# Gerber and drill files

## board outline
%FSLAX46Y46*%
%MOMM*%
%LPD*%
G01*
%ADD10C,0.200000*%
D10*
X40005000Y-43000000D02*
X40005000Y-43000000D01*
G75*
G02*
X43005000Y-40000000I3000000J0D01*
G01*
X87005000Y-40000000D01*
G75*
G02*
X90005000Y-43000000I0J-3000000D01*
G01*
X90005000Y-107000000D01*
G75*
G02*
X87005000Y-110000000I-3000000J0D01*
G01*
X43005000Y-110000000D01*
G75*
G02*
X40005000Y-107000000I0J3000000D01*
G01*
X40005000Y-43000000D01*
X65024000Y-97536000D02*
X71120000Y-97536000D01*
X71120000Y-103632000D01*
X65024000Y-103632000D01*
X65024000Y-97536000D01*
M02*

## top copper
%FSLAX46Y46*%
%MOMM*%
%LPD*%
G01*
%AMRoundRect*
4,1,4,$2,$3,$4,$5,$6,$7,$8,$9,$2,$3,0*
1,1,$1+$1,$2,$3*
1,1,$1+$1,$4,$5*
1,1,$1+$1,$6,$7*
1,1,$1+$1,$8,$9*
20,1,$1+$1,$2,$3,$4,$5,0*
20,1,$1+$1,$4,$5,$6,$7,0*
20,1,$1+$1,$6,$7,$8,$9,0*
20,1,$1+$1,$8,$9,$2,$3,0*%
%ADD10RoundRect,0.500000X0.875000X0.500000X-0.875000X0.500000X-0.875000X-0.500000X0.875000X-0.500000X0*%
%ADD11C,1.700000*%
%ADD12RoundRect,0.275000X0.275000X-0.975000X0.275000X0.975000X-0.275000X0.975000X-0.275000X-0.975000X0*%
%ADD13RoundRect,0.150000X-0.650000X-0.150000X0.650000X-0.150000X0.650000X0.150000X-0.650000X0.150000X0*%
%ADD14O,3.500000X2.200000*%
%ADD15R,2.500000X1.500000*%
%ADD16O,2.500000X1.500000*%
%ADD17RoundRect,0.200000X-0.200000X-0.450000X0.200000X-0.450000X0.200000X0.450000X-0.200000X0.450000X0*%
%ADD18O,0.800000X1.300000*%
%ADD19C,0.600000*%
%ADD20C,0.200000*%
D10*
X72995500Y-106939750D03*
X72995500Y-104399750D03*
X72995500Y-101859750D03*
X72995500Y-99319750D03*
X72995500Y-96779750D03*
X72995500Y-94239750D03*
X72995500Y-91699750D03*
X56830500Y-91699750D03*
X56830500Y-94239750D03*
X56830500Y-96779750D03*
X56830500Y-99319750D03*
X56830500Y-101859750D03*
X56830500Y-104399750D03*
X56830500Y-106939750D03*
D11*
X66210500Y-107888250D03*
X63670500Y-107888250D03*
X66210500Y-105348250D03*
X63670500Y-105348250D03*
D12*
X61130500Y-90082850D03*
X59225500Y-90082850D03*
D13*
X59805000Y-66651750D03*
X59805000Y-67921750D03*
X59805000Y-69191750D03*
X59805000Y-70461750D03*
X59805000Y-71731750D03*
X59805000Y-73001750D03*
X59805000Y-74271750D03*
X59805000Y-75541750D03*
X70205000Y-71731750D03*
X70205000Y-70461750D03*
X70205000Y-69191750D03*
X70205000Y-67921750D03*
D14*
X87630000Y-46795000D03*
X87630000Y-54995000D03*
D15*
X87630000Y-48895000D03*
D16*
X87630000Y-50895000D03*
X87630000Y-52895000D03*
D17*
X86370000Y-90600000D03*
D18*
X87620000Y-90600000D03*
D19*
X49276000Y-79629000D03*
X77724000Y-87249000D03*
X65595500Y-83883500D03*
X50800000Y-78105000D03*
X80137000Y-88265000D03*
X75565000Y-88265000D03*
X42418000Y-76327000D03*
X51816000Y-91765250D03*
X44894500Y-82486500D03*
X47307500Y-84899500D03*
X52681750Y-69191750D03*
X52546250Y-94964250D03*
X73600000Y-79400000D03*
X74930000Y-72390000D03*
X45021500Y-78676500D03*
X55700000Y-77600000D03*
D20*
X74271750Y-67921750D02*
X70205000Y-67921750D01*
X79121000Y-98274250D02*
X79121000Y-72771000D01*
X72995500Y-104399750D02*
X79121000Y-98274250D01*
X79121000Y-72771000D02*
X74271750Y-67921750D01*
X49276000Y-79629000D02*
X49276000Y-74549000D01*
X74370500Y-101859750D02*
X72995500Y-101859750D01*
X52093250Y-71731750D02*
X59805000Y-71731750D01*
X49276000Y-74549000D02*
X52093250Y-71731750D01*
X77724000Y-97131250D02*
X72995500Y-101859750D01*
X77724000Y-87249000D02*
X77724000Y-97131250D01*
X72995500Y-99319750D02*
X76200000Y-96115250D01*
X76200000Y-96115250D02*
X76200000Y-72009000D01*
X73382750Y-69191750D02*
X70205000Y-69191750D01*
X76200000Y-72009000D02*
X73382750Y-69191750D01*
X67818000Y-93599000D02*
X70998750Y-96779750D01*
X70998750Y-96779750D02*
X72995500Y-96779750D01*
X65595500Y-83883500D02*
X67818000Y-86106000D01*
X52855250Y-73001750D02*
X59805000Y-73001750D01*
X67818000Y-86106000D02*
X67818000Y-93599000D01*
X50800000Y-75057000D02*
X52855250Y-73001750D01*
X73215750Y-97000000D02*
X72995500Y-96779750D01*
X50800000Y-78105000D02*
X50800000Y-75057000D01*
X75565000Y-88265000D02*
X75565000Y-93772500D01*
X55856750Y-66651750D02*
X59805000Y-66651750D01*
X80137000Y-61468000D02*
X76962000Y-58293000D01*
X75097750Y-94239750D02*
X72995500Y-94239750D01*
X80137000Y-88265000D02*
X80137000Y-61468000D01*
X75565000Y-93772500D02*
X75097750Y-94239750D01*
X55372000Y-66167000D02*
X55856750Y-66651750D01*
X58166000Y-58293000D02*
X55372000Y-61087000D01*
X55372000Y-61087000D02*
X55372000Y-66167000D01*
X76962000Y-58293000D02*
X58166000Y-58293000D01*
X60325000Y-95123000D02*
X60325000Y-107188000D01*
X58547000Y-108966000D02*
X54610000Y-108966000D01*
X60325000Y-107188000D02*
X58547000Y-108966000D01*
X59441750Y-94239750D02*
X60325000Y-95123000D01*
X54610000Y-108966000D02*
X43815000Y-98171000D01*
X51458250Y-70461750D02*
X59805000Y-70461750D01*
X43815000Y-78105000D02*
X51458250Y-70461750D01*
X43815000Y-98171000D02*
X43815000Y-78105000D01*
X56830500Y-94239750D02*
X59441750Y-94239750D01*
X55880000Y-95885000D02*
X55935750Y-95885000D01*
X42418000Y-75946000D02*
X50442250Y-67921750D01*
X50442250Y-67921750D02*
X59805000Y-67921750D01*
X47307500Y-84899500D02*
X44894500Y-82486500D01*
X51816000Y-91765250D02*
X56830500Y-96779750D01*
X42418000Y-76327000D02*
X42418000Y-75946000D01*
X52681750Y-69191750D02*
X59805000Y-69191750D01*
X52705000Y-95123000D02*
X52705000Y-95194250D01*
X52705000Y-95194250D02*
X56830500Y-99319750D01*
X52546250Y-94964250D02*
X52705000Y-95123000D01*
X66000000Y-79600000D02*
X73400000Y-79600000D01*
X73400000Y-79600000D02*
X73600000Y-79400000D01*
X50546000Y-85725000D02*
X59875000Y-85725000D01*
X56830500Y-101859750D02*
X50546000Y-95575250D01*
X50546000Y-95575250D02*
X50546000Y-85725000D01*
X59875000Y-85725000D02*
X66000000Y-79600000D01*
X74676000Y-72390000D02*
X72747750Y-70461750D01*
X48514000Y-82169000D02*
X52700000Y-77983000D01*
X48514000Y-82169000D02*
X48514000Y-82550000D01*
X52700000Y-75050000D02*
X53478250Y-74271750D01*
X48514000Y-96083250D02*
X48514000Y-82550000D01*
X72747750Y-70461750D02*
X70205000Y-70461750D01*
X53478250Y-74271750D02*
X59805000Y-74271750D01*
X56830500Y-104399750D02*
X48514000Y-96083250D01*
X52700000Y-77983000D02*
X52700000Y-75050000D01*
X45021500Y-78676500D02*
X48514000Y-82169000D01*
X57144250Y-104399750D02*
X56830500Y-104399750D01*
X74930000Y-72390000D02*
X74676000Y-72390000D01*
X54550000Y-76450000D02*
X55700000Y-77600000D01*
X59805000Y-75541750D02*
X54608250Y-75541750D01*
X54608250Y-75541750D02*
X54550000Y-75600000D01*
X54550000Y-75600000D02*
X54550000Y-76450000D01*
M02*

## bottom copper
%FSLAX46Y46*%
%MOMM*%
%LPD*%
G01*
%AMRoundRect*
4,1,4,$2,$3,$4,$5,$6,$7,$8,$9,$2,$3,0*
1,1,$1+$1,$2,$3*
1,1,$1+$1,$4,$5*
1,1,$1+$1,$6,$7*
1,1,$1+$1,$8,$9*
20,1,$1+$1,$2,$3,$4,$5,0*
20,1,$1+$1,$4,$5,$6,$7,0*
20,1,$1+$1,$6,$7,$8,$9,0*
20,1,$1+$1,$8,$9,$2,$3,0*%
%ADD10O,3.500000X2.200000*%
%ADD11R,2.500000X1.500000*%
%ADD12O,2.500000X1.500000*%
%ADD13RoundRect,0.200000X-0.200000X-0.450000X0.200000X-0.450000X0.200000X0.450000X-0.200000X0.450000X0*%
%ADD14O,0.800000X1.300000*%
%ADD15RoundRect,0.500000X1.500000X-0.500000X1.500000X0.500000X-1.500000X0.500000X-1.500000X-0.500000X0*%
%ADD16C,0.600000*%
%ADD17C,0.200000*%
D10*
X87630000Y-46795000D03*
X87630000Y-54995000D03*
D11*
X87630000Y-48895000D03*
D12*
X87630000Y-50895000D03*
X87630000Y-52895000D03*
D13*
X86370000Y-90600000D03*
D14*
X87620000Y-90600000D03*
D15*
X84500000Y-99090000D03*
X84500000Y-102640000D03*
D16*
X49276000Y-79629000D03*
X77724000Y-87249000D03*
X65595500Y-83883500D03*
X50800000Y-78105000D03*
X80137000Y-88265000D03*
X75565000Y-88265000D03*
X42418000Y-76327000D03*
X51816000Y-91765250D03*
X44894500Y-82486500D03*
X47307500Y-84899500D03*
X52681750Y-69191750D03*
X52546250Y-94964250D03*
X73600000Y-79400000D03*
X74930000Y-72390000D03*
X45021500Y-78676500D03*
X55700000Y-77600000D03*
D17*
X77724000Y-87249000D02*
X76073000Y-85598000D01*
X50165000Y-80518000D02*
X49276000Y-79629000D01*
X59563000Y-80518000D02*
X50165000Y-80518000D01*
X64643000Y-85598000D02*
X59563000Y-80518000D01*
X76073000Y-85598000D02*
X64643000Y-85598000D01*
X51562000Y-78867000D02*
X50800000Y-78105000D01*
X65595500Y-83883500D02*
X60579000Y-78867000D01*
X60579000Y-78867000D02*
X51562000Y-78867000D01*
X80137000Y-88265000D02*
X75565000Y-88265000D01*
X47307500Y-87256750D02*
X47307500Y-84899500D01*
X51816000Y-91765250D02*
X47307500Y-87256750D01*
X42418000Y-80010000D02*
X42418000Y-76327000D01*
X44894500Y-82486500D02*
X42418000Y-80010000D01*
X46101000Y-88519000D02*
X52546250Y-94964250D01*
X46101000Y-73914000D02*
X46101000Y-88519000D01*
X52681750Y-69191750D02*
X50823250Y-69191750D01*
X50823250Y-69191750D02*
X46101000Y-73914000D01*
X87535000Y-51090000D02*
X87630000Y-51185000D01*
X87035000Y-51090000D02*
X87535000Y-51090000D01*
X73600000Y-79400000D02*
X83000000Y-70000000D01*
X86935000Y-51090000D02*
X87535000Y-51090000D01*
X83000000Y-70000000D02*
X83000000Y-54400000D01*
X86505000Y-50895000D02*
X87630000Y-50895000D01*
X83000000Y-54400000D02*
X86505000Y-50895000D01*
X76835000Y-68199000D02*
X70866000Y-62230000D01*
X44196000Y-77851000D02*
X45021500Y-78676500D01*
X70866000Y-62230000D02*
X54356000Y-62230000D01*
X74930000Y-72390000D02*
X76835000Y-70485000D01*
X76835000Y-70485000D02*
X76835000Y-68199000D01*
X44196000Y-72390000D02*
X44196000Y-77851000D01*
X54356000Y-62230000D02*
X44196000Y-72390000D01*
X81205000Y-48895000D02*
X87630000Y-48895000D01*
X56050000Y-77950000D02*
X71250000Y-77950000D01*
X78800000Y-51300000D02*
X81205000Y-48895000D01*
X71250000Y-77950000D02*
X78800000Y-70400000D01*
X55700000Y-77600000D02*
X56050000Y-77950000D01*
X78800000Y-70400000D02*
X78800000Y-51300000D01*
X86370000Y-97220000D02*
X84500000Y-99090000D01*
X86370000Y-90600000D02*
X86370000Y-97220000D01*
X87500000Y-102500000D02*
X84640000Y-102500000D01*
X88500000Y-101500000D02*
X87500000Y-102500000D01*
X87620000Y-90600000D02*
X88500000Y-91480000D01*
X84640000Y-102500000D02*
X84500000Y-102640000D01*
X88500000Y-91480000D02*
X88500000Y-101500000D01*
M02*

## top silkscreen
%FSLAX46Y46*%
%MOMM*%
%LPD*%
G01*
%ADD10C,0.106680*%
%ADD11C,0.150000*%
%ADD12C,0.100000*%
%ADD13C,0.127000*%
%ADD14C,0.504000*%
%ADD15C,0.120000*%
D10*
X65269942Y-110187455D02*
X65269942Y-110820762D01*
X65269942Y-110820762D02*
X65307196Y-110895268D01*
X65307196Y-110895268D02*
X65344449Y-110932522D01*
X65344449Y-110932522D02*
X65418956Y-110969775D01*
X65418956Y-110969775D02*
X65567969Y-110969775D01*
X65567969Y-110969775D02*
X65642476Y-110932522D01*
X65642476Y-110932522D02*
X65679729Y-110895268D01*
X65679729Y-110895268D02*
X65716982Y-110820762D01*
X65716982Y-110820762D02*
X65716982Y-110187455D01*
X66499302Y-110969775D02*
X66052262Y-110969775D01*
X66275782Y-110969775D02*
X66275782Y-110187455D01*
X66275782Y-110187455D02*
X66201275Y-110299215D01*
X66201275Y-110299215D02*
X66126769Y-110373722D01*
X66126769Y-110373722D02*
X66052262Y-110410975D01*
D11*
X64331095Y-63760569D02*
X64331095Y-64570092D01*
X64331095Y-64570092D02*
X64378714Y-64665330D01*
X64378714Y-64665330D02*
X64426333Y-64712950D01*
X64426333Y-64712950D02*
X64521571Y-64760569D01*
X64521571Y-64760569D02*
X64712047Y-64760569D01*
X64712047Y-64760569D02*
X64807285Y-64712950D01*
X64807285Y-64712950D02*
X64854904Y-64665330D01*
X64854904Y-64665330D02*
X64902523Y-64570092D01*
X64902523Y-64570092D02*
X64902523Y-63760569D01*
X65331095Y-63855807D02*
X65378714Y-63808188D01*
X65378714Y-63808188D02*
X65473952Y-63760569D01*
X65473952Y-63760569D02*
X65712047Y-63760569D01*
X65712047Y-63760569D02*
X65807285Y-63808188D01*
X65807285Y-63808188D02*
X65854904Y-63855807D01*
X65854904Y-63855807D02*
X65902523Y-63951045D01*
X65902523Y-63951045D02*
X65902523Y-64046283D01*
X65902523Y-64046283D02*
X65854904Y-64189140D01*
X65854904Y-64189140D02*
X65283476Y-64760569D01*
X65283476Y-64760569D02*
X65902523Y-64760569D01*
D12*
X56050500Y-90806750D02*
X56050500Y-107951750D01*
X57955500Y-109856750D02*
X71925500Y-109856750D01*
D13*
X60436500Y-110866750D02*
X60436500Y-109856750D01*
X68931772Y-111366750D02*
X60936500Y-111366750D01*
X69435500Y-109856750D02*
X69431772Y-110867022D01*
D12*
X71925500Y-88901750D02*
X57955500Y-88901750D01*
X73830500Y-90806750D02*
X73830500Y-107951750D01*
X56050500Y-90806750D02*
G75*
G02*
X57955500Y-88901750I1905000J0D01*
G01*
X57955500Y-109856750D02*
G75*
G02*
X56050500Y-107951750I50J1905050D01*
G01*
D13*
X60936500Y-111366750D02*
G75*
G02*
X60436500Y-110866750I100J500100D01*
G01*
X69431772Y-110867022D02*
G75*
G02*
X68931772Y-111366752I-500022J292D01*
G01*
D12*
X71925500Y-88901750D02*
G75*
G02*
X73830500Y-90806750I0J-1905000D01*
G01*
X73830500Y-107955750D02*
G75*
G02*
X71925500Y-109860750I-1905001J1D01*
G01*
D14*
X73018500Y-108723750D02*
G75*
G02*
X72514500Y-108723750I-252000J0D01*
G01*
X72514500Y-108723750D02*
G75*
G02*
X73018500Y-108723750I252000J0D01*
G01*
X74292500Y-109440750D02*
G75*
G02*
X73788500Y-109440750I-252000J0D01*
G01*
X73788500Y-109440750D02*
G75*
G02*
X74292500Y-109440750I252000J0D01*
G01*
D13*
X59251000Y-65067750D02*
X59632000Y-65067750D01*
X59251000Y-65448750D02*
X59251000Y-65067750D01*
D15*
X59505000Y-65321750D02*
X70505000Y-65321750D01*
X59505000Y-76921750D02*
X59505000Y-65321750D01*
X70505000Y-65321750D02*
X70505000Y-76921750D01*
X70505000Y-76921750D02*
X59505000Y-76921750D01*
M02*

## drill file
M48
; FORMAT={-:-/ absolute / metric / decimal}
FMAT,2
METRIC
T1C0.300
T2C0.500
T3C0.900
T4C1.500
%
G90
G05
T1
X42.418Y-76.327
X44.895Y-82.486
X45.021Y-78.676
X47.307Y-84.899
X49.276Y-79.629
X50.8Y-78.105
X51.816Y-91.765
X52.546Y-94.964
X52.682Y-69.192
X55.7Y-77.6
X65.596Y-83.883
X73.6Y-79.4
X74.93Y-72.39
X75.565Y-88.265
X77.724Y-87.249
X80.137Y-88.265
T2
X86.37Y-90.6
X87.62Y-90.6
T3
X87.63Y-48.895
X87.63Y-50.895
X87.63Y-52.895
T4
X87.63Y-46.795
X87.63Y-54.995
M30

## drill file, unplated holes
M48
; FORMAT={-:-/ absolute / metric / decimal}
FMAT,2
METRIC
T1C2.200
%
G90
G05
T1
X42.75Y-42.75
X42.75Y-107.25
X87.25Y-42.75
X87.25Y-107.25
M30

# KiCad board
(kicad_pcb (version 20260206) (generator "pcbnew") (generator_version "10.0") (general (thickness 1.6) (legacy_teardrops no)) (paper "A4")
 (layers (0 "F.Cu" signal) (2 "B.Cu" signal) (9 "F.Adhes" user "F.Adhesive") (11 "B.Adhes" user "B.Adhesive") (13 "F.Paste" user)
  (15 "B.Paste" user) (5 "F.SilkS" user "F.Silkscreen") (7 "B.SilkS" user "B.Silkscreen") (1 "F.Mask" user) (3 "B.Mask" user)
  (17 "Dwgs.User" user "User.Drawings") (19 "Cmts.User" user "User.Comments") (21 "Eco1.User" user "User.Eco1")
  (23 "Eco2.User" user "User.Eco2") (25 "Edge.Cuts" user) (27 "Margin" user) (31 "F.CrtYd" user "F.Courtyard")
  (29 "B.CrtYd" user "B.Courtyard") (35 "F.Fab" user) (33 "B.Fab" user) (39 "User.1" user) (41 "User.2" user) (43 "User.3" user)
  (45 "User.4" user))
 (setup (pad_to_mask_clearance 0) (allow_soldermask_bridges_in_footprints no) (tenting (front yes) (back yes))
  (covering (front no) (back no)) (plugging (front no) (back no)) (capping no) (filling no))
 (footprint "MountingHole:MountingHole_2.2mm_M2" (layer "F.Cu") (at 87.25 42.75)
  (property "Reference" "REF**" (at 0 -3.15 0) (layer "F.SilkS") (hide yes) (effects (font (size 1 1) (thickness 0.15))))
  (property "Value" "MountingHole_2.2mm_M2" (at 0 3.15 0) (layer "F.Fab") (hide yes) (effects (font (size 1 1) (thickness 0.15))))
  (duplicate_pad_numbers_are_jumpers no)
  (pad "" np_thru_hole circle (at 0 0) (size 2.2 2.2) (drill 2.2) (layers "*.Cu" "*.Mask")))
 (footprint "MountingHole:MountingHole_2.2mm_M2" (layer "F.Cu") (at 42.75 42.75)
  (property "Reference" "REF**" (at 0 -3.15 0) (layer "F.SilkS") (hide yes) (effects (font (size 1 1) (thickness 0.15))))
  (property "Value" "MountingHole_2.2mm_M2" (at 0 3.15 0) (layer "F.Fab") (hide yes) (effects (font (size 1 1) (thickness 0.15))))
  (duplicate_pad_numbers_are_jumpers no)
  (pad "" np_thru_hole circle (at 0 0) (size 2.2 2.2) (drill 2.2) (layers "*.Cu" "*.Mask")))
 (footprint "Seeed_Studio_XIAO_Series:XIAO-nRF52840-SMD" (layer "F.Cu") (at 73.8305 88.81975 180)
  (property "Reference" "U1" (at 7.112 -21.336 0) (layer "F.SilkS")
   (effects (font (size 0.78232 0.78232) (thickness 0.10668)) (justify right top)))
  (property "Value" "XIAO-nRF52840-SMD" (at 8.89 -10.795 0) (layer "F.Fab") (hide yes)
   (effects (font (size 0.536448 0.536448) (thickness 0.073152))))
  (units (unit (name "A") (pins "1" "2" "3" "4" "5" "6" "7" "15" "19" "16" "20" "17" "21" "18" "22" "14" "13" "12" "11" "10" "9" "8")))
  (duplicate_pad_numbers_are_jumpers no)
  (fp_line (start 17.78 -1.987) (end 17.78 -19.132) (stroke (width 0.1) (type solid)) (layer "F.SilkS"))
  (fp_line (start 15.875 -21.037) (end 1.905 -21.037) (stroke (width 0.1) (type solid)) (layer "F.SilkS"))
  (fp_line (start 13.394 -22.047) (end 13.394 -21.037) (stroke (width 0.127) (type solid)) (layer "F.SilkS"))
  (fp_line (start 4.898728 -22.547) (end 12.894 -22.547) (stroke (width 0.127) (type solid)) (layer "F.SilkS"))
  (fp_line (start 4.395 -21.037) (end 4.398728 -22.047272) (stroke (width 0.127) (type solid)) (layer "F.SilkS"))
  (fp_line (start 1.905 -0.082) (end 15.875 -0.082) (stroke (width 0.1) (type solid)) (layer "F.SilkS"))
  (fp_line (start 0 -1.987) (end 0 -19.132) (stroke (width 0.1) (type solid)) (layer "F.SilkS"))
  (fp_arc (start 17.78 -1.987) (mid 17.222038 -0.639961) (end 15.875 -0.082) (stroke (width 0.1) (type solid)) (layer "F.SilkS"))
  (fp_arc (start 15.875 -21.037) (mid 17.222016 -20.479031) (end 17.78 -19.132) (stroke (width 0.1) (type solid)) (layer "F.SilkS"))
  (fp_arc (start 12.894 -22.547) (mid 13.247531 -22.400546) (end 13.394 -22.047) (stroke (width 0.127) (type default)) (layer "F.SilkS"))
  (fp_arc (start 4.398728 -22.047272) (mid 4.545276 -22.400644) (end 4.898728 -22.547) (stroke (width 0.127) (type default))
   (layer "F.SilkS"))
  (fp_arc (start 1.905 -0.082) (mid 0.557962 -0.639962) (end 0 -1.987) (stroke (width 0.1) (type solid)) (layer "F.SilkS"))
  (fp_arc (start 0 -19.136) (mid 0.557962 -20.483038) (end 1.905 -21.041) (stroke (width 0.1) (type solid)) (layer "F.SilkS"))
  (fp_circle (center 1.064 -19.904) (end 1.064 -20.158) (stroke (width 0.5) (type solid)) (fill yes) (layer "F.SilkS"))
  (fp_circle (center -0.21 -20.621) (end -0.21 -20.875) (stroke (width 0.5) (type solid)) (fill yes) (layer "F.SilkS"))
  (pad "1" smd roundrect (at 0.835 -18.12 180) (size 2.75 2) (layers "F.Cu" "F.Mask" "F.Paste") (roundrect_rratio 0.25)
   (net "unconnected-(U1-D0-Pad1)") (solder_mask_margin 0.0508) (thermal_bridge_angle 45))
  (pad "2" smd roundrect (at 0.835 -15.58 180) (size 2.75 2) (layers "F.Cu" "F.Mask" "F.Paste") (roundrect_rratio 0.25) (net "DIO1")
   (solder_mask_margin 0.0508) (thermal_bridge_angle 45))
  (pad "3" smd roundrect (at 0.835 -13.04 180) (size 2.75 2) (layers "F.Cu" "F.Mask" "F.Paste") (roundrect_rratio 0.25) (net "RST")
   (solder_mask_margin 0.0508) (thermal_bridge_angle 45))
  (pad "4" smd roundrect (at 0.835 -10.5 180) (size 2.75 2) (layers "F.Cu" "F.Mask" "F.Paste") (roundrect_rratio 0.25) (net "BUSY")
   (solder_mask_margin 0.0508) (thermal_bridge_angle 45))
  (pad "5" smd roundrect (at 0.835 -7.96 180) (size 2.75 2) (layers "F.Cu" "F.Mask" "F.Paste") (roundrect_rratio 0.25) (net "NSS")
   (solder_mask_margin 0.0508) (thermal_bridge_angle 45))
  (pad "6" smd roundrect (at 0.835 -5.42 180) (size 2.75 2) (layers "F.Cu" "F.Mask" "F.Paste") (roundrect_rratio 0.25) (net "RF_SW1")
   (solder_mask_margin 0.0508) (thermal_bridge_angle 45))
  (pad "7" smd roundrect (at 0.835 -2.88 180) (size 2.75 2) (layers "F.Cu" "F.Mask" "F.Paste") (roundrect_rratio 0.25)
   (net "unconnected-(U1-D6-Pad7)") (solder_mask_margin 0.0508) (thermal_bridge_angle 45))
  (pad "8" smd roundrect (at 17 -2.88 180) (size 2.75 2) (layers "F.Cu" "F.Mask" "F.Paste") (roundrect_rratio 0.25)
   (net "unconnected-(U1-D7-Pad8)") (solder_mask_margin 0.0508) (thermal_bridge_angle 45))
  (pad "9" smd roundrect (at 17 -5.42 180) (size 2.75 2) (layers "F.Cu" "F.Mask" "F.Paste") (roundrect_rratio 0.25) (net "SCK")
   (solder_mask_margin 0.0508) (thermal_bridge_angle 45))
  (pad "10" smd roundrect (at 17 -7.96 180) (size 2.75 2) (layers "F.Cu" "F.Mask" "F.Paste") (roundrect_rratio 0.25) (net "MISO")
   (solder_mask_margin 0.0508) (thermal_bridge_angle 45))
  (pad "11" smd roundrect (at 17 -10.5 180) (size 2.75 2) (layers "F.Cu" "F.Mask" "F.Paste") (roundrect_rratio 0.25) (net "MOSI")
   (solder_mask_margin 0.0508) (thermal_bridge_angle 45))
  (pad "12" smd roundrect (at 17 -13.04 180) (size 2.75 2) (layers "F.Cu" "F.Mask" "F.Paste") (roundrect_rratio 0.25) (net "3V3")
   (solder_mask_margin 0.0508) (thermal_bridge_angle 45))
  (pad "13" smd roundrect (at 17 -15.58 180) (size 2.75 2) (layers "F.Cu" "F.Mask" "F.Paste") (roundrect_rratio 0.25) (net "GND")
   (solder_mask_margin 0.0508) (thermal_bridge_angle 45))
  (pad "14" smd roundrect (at 17 -18.12 180) (size 2.75 2) (layers "F.Cu" "F.Mask" "F.Paste") (roundrect_rratio 0.25)
   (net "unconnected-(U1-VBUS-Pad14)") (solder_mask_margin 0.0508) (thermal_bridge_angle 45))
  (pad "15" smd circle (at 7.62 -19.0685 180) (size 1.7 1.7) (layers "F.Cu" "F.Mask" "F.Paste") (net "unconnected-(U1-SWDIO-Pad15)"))
  (pad "16" smd circle (at 10.16 -19.0685 180) (size 1.7 1.7) (layers "F.Cu" "F.Mask" "F.Paste") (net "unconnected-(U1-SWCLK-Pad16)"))
  (pad "17" smd circle (at 7.62 -16.5285 180) (size 1.7 1.7) (layers "F.Cu" "F.Mask" "F.Paste") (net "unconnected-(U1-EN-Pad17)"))
  (pad "18" smd circle (at 10.16 -16.5285 180) (size 1.7 1.7) (layers "F.Cu" "F.Mask" "F.Paste") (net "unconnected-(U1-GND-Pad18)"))
  (pad "21" smd roundrect (at 12.7 -1.2631 90) (size 2.5 1.1) (layers "F.Cu" "F.Mask" "F.Paste") (roundrect_rratio 0.25)
   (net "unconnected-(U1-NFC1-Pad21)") (thermal_bridge_angle 45))
  (pad "22" smd roundrect (at 14.605 -1.2631 90) (size 2.5 1.1) (layers "F.Cu" "F.Mask" "F.Paste") (roundrect_rratio 0.25)
   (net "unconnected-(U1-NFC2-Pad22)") (thermal_bridge_angle 45)))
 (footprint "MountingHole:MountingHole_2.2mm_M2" (layer "F.Cu") (at 42.75 107.25)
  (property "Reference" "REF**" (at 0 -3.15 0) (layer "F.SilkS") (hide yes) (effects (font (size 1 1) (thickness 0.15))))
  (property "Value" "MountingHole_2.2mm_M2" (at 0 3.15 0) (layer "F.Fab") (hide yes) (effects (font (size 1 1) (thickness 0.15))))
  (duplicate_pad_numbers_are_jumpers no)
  (pad "" np_thru_hole circle (at 0 0) (size 2.2 2.2) (drill 2.2) (layers "*.Cu" "*.Mask")))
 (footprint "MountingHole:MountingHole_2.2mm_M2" (layer "F.Cu") (at 87.25 107.25)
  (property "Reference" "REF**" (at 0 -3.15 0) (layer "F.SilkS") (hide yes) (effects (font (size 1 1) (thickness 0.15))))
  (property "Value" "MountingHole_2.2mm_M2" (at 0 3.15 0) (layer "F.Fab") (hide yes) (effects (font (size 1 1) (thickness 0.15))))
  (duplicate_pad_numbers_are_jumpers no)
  (pad "" np_thru_hole circle (at 0 0) (size 2.2 2.2) (drill 2.2) (layers "*.Cu" "*.Mask")))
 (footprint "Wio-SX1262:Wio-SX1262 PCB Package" (layer "F.Cu") (at 59.505 65.32175 -90)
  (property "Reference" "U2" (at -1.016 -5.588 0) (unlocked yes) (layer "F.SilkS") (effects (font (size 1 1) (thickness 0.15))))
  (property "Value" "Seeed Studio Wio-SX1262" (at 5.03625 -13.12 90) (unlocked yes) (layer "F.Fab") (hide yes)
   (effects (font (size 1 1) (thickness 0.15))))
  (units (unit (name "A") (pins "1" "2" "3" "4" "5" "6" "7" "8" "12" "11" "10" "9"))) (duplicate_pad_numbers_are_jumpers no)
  (fp_line (start -0.254 0.254) (end -0.254 -0.127) (stroke (width 0.127) (type default)) (layer "F.SilkS"))
  (fp_line (start 0.127 0.254) (end -0.254 0.254) (stroke (width 0.127) (type default)) (layer "F.SilkS"))
  (fp_line (start 0 0) (end 0 -11) (stroke (width 0.12) (type default)) (layer "F.SilkS"))
  (fp_line (start 11.6 0) (end 0 0) (stroke (width 0.12) (type default)) (layer "F.SilkS"))
  (fp_line (start 0 -11) (end 11.6 -11) (stroke (width 0.12) (type default)) (layer "F.SilkS"))
  (fp_line (start 11.6 -11) (end 11.6 0) (stroke (width 0.12) (type default)) (layer "F.SilkS"))
  (pad "1" smd roundrect (at 1.33 -0.3) (size 1.6 0.6) (layers "F.Cu" "F.Mask" "F.Paste") (roundrect_rratio 0.25) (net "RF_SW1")
   (thermal_bridge_angle 45))
  (pad "2" smd roundrect (at 2.6 -0.3) (size 1.6 0.6) (layers "F.Cu" "F.Mask" "F.Paste") (roundrect_rratio 0.25) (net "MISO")
   (thermal_bridge_angle 45))
  (pad "3" smd roundrect (at 3.87 -0.3) (size 1.6 0.6) (layers "F.Cu" "F.Mask" "F.Paste") (roundrect_rratio 0.25) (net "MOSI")
   (thermal_bridge_angle 45))
  (pad "4" smd roundrect (at 5.14 -0.3) (size 1.6 0.6) (layers "F.Cu" "F.Mask" "F.Paste") (roundrect_rratio 0.25) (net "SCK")
   (thermal_bridge_angle 45))
  (pad "5" smd roundrect (at 6.41 -0.3) (size 1.6 0.6) (layers "F.Cu" "F.Mask" "F.Paste") (roundrect_rratio 0.25) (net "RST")
   (thermal_bridge_angle 45))
  (pad "6" smd roundrect (at 7.68 -0.3) (size 1.6 0.6) (layers "F.Cu" "F.Mask" "F.Paste") (roundrect_rratio 0.25) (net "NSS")
   (thermal_bridge_angle 45))
  (pad "7" smd roundrect (at 8.95 -0.3) (size 1.6 0.6) (layers "F.Cu" "F.Mask" "F.Paste") (roundrect_rratio 0.25) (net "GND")
   (thermal_bridge_angle 45))
  (pad "8" smd roundrect (at 10.22 -0.3) (size 1.6 0.6) (layers "F.Cu" "F.Mask" "F.Paste") (roundrect_rratio 0.25) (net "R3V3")
   (thermal_bridge_angle 45))
  (pad "9" smd roundrect (at 6.41 -10.7) (size 1.6 0.6) (layers "F.Cu" "F.Mask" "F.Paste") (roundrect_rratio 0.25)
   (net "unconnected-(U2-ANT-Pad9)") (thermal_bridge_angle 45))
  (pad "10" smd roundrect (at 5.14 -10.7) (size 1.6 0.6) (layers "F.Cu" "F.Mask" "F.Paste") (roundrect_rratio 0.25) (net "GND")
   (thermal_bridge_angle 45))
  (pad "11" smd roundrect (at 3.87 -10.7) (size 1.6 0.6) (layers "F.Cu" "F.Mask" "F.Paste") (roundrect_rratio 0.25) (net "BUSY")
   (thermal_bridge_angle 45))
  (pad "12" smd roundrect (at 2.6 -10.7) (size 1.6 0.6) (layers "F.Cu" "F.Mask" "F.Paste") (roundrect_rratio 0.25) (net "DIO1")
   (thermal_bridge_angle 45)))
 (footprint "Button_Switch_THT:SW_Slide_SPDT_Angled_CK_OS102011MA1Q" (layer "B.Cu") (at 87.63 48.895 -90)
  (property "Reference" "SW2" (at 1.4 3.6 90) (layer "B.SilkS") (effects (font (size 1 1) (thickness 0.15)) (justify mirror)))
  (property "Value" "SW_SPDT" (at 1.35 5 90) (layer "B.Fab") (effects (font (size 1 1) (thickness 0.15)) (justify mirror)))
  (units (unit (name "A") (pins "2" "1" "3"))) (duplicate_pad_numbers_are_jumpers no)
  (pad "" thru_hole oval (at -2.1 0 270) (size 2.2 3.5) (drill 1.5) (layers "*.Cu" "*.Mask") (remove_unused_layers no))
  (pad "" thru_hole oval (at 6.1 0 270) (size 2.2 3.5) (drill 1.5) (layers "*.Cu" "*.Mask") (remove_unused_layers no))
  (pad "1" thru_hole rect (at 0 0 270) (size 1.5 2.5) (drill 0.9) (layers "*.Cu" "*.Mask") (remove_unused_layers no) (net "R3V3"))
  (pad "2" thru_hole oval (at 2 0 270) (size 1.5 2.5) (drill 0.9) (layers "*.Cu" "*.Mask") (remove_unused_layers no) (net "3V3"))
  (pad "3" thru_hole oval (at 4 0 270) (size 1.5 2.5) (drill 0.9) (layers "*.Cu" "*.Mask") (remove_unused_layers no)
   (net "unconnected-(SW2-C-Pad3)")))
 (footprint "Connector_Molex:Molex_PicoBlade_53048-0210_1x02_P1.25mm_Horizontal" (layer "B.Cu") (at 86.37 90.6)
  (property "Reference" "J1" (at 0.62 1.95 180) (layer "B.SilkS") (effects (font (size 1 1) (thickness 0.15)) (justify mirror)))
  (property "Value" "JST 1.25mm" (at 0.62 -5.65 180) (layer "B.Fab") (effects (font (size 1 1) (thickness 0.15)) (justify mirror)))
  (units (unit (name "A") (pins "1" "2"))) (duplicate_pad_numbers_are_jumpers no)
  (pad "1" thru_hole roundrect (at 0 0) (size 0.8 1.3) (drill 0.5) (layers "*.Cu" "*.Mask") (remove_unused_layers no)
   (roundrect_rratio 0.25) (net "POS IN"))
  (pad "2" thru_hole oval (at 1.25 0) (size 0.8 1.3) (drill 0.5) (layers "*.Cu" "*.Mask") (remove_unused_layers no) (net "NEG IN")))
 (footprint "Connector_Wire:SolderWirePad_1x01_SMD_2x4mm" (layer "B.Cu") (at 84.5 99.09 90)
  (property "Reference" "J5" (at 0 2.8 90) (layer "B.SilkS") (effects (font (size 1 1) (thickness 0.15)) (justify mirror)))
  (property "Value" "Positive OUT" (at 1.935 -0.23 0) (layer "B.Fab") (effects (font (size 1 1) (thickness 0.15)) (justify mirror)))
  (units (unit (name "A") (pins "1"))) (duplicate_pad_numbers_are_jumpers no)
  (pad "1" smd roundrect (at 0 0 90) (size 2 4) (layers "B.Cu" "B.Mask") (roundrect_rratio 0.25) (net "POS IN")))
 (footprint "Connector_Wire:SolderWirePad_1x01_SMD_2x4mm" (layer "B.Cu") (at 84.5 102.64 90)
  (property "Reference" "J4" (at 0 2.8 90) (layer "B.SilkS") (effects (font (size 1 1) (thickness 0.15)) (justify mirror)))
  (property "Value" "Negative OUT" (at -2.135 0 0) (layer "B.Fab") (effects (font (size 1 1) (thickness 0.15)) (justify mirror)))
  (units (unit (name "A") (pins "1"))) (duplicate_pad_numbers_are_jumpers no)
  (pad "1" smd roundrect (at 0 0 90) (size 2 4) (layers "B.Cu" "B.Mask") (roundrect_rratio 0.25) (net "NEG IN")))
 (gr_rect (start 40.005 40) (end 90.005 110) (radius 3) (stroke (width 0.2) (type solid)) (fill no) (layer "Edge.Cuts"))
 (gr_rect (start 65.024 97.536) (end 71.12 103.632) (stroke (width 0.2) (type default)) (fill no) (layer "Edge.Cuts"))
 (segment (start 74.27175 67.92175) (end 70.205 67.92175) (width 0.2) (layer "F.Cu") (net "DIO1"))
 (segment (start 79.121 98.27425) (end 79.121 72.771) (width 0.2) (layer "F.Cu") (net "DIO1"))
 (segment (start 72.9955 104.39975) (end 79.121 98.27425) (width 0.2) (layer "F.Cu") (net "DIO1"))
 (segment (start 79.121 72.771) (end 74.27175 67.92175) (width 0.2) (layer "F.Cu") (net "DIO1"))
 (segment (start 49.276 79.629) (end 49.276 74.549) (width 0.2) (layer "F.Cu") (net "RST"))
 (segment (start 74.3705 101.85975) (end 72.9955 101.85975) (width 0.2) (layer "F.Cu") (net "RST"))
 (segment (start 52.09325 71.73175) (end 59.805 71.73175) (width 0.2) (layer "F.Cu") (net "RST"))
 (segment (start 49.276 74.549) (end 52.09325 71.73175) (width 0.2) (layer "F.Cu") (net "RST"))
 (segment (start 77.724 97.13125) (end 72.9955 101.85975) (width 0.2) (layer "F.Cu") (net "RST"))
 (segment (start 77.724 87.249) (end 77.724 97.13125) (width 0.2) (layer "F.Cu") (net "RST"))
 (via (at 49.276 79.629) (size 0.6) (drill 0.3) (layers "F.Cu" "B.Cu") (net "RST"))
 (via (at 77.724 87.249) (size 0.6) (drill 0.3) (layers "F.Cu" "B.Cu") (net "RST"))
 (segment (start 77.724 87.249) (end 76.073 85.598) (width 0.2) (layer "B.Cu") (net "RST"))
 (segment (start 50.165 80.518) (end 49.276 79.629) (width 0.2) (layer "B.Cu") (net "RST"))
 (segment (start 59.563 80.518) (end 50.165 80.518) (width 0.2) (layer "B.Cu") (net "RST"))
 (segment (start 64.643 85.598) (end 59.563 80.518) (width 0.2) (layer "B.Cu") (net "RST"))
 (segment (start 76.073 85.598) (end 64.643 85.598) (width 0.2) (layer "B.Cu") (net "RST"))
 (segment (start 72.9955 99.31975) (end 76.2 96.11525) (width 0.2) (layer "F.Cu") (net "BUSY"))
 (segment (start 76.2 96.11525) (end 76.2 72.009) (width 0.2) (layer "F.Cu") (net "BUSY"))
 (segment (start 73.38275 69.19175) (end 70.205 69.19175) (width 0.2) (layer "F.Cu") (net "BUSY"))
 (segment (start 76.2 72.009) (end 73.38275 69.19175) (width 0.2) (layer "F.Cu") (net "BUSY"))
 (segment (start 67.818 93.599) (end 70.99875 96.77975) (width 0.2) (layer "F.Cu") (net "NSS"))
 (segment (start 70.99875 96.77975) (end 72.9955 96.77975) (width 0.2) (layer "F.Cu") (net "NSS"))
 (segment (start 65.5955 83.8835) (end 67.818 86.106) (width 0.2) (layer "F.Cu") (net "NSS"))
 (segment (start 52.85525 73.00175) (end 59.805 73.00175) (width 0.2) (layer "F.Cu") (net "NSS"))
 (segment (start 67.818 86.106) (end 67.818 93.599) (width 0.2) (layer "F.Cu") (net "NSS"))
 (segment (start 50.8 75.057) (end 52.85525 73.00175) (width 0.2) (layer "F.Cu") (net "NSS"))
 (segment (start 73.21575 97) (end 72.9955 96.77975) (width 0.2) (layer "F.Cu") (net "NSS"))
 (segment (start 50.8 78.105) (end 50.8 75.057) (width 0.2) (layer "F.Cu") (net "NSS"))
 (via (at 65.5955 83.8835) (size 0.6) (drill 0.3) (layers "F.Cu" "B.Cu") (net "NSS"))
 (via (at 50.8 78.105) (size 0.6) (drill 0.3) (layers "F.Cu" "B.Cu") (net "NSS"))
 (segment (start 51.562 78.867) (end 50.8 78.105) (width 0.2) (layer "B.Cu") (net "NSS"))
 (segment (start 65.5955 83.8835) (end 60.579 78.867) (width 0.2) (layer "B.Cu") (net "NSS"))
 (segment (start 60.579 78.867) (end 51.562 78.867) (width 0.2) (layer "B.Cu") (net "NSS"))
 (segment (start 75.565 88.265) (end 75.565 93.7725) (width 0.2) (layer "F.Cu") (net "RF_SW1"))
 (segment (start 55.85675 66.65175) (end 59.805 66.65175) (width 0.2) (layer "F.Cu") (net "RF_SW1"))
 (segment (start 80.137 61.468) (end 76.962 58.293) (width 0.2) (layer "F.Cu") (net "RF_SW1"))
 (segment (start 75.09775 94.23975) (end 72.9955 94.23975) (width 0.2) (layer "F.Cu") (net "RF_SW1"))
 (segment (start 80.137 88.265) (end 80.137 61.468) (width 0.2) (layer "F.Cu") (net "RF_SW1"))
 (segment (start 75.565 93.7725) (end 75.09775 94.23975) (width 0.2) (layer "F.Cu") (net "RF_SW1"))
 (segment (start 55.372 66.167) (end 55.85675 66.65175) (width 0.2) (layer "F.Cu") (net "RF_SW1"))
 (segment (start 58.166 58.293) (end 55.372 61.087) (width 0.2) (layer "F.Cu") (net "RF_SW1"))
 (segment (start 55.372 61.087) (end 55.372 66.167) (width 0.2) (layer "F.Cu") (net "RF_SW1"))
 (segment (start 76.962 58.293) (end 58.166 58.293) (width 0.2) (layer "F.Cu") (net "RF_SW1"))
 (via (at 80.137 88.265) (size 0.6) (drill 0.3) (layers "F.Cu" "B.Cu") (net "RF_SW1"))
 (via (at 75.565 88.265) (size 0.6) (drill 0.3) (layers "F.Cu" "B.Cu") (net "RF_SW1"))
 (segment (start 80.137 88.265) (end 75.565 88.265) (width 0.2) (layer "B.Cu") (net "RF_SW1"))
 (segment (start 60.325 95.123) (end 60.325 107.188) (width 0.2) (layer "F.Cu") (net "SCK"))
 (segment (start 58.547 108.966) (end 54.61 108.966) (width 0.2) (layer "F.Cu") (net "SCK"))
 (segment (start 60.325 107.188) (end 58.547 108.966) (width 0.2) (layer "F.Cu") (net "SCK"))
 (segment (start 59.44175 94.23975) (end 60.325 95.123) (width 0.2) (layer "F.Cu") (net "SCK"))
 (segment (start 54.61 108.966) (end 43.815 98.171) (width 0.2) (layer "F.Cu") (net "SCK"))
 (segment (start 51.45825 70.46175) (end 59.805 70.46175) (width 0.2) (layer "F.Cu") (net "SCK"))
 (segment (start 43.815 78.105) (end 51.45825 70.46175) (width 0.2) (layer "F.Cu") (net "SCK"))
 (segment (start 43.815 98.171) (end 43.815 78.105) (width 0.2) (layer "F.Cu") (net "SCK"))
 (segment (start 56.8305 94.23975) (end 59.44175 94.23975) (width 0.2) (layer "F.Cu") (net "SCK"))
 (segment (start 55.88 95.885) (end 55.93575 95.885) (width 0.2) (layer "F.Cu") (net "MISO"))
 (segment (start 42.418 75.946) (end 50.44225 67.92175) (width 0.2) (layer "F.Cu") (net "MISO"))
 (segment (start 50.44225 67.92175) (end 59.805 67.92175) (width 0.2) (layer "F.Cu") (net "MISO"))
 (segment (start 47.3075 84.8995) (end 44.8945 82.4865) (width 0.2) (layer "F.Cu") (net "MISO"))
 (segment (start 51.816 91.76525) (end 56.8305 96.77975) (width 0.2) (layer "F.Cu") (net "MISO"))
 (segment (start 42.418 76.327) (end 42.418 75.946) (width 0.2) (layer "F.Cu") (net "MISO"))
 (via (at 42.418 76.327) (size 0.6) (drill 0.3) (layers "F.Cu" "B.Cu") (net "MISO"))
 (via (at 51.816 91.76525) (size 0.6) (drill 0.3) (layers "F.Cu" "B.Cu") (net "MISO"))
 (via (at 44.8945 82.4865) (size 0.6) (drill 0.3) (layers "F.Cu" "B.Cu") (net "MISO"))
 (via (at 47.3075 84.8995) (size 0.6) (drill 0.3) (layers "F.Cu" "B.Cu") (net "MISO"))
 (segment (start 47.3075 87.25675) (end 47.3075 84.8995) (width 0.2) (layer "B.Cu") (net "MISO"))
 (segment (start 51.816 91.76525) (end 47.3075 87.25675) (width 0.2) (layer "B.Cu") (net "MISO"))
 (segment (start 42.418 80.01) (end 42.418 76.327) (width 0.2) (layer "B.Cu") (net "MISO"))
 (segment (start 44.8945 82.4865) (end 42.418 80.01) (width 0.2) (layer "B.Cu") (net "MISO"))
 (segment (start 52.68175 69.19175) (end 59.805 69.19175) (width 0.2) (layer "F.Cu") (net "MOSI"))
 (segment (start 52.705 95.123) (end 52.705 95.19425) (width 0.2) (layer "F.Cu") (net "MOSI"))
 (segment (start 52.705 95.19425) (end 56.8305 99.31975) (width 0.2) (layer "F.Cu") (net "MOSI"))
 (segment (start 52.54625 94.96425) (end 52.705 95.123) (width 0.2) (layer "F.Cu") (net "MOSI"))
 (via (at 52.68175 69.19175) (size 0.6) (drill 0.3) (layers "F.Cu" "B.Cu") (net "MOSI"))
 (via (at 52.54625 94.96425) (size 0.6) (drill 0.3) (layers "F.Cu" "B.Cu") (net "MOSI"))
 (segment (start 46.101 88.519) (end 52.54625 94.96425) (width 0.2) (layer "B.Cu") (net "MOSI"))
 (segment (start 46.101 73.914) (end 46.101 88.519) (width 0.2) (layer "B.Cu") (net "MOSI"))
 (segment (start 52.68175 69.19175) (end 50.82325 69.19175) (width 0.2) (layer "B.Cu") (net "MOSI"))
 (segment (start 50.82325 69.19175) (end 46.101 73.914) (width 0.2) (layer "B.Cu") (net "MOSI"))
 (segment (start 66 79.6) (end 73.4 79.6) (width 0.2) (layer "F.Cu") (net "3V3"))
 (segment (start 73.4 79.6) (end 73.6 79.4) (width 0.2) (layer "F.Cu") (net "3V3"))
 (segment (start 50.546 85.725) (end 59.875 85.725) (width 0.2) (layer "F.Cu") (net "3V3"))
 (segment (start 56.8305 101.85975) (end 50.546 95.57525) (width 0.2) (layer "F.Cu") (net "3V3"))
 (segment (start 50.546 95.57525) (end 50.546 85.725) (width 0.2) (layer "F.Cu") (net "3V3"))
 (segment (start 59.875 85.725) (end 66 79.6) (width 0.2) (layer "F.Cu") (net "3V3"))
 (via (at 73.6 79.4) (size 0.6) (drill 0.3) (layers "F.Cu" "B.Cu") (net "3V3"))
 (segment (start 87.535 51.09) (end 87.63 51.185) (width 0.2) (layer "B.Cu") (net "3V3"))
 (segment (start 87.035 51.09) (end 87.535 51.09) (width 0.2) (layer "B.Cu") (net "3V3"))
 (segment (start 73.6 79.4) (end 83 70) (width 0.2) (layer "B.Cu") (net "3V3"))
 (segment (start 86.935 51.09) (end 87.535 51.09) (width 0.2) (layer "B.Cu") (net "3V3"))
 (segment (start 83 70) (end 83 54.4) (width 0.2) (layer "B.Cu") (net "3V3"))
 (segment (start 86.505 50.895) (end 87.63 50.895) (width 0.2) (layer "B.Cu") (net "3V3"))
 (segment (start 83 54.4) (end 86.505 50.895) (width 0.2) (layer "B.Cu") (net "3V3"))
 (segment (start 74.676 72.39) (end 72.74775 70.46175) (width 0.2) (layer "F.Cu") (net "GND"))
 (segment (start 48.514 82.169) (end 52.7 77.983) (width 0.2) (layer "F.Cu") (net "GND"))
 (segment (start 48.514 82.169) (end 48.514 82.55) (width 0.2) (layer "F.Cu") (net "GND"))
 (segment (start 52.7 75.05) (end 53.47825 74.27175) (width 0.2) (layer "F.Cu") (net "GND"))
 (segment (start 48.514 96.08325) (end 48.514 82.55) (width 0.2) (layer "F.Cu") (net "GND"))
 (segment (start 72.74775 70.46175) (end 70.205 70.46175) (width 0.2) (layer "F.Cu") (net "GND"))
 (segment (start 53.47825 74.27175) (end 59.805 74.27175) (width 0.2) (layer "F.Cu") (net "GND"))
 (segment (start 56.8305 104.39975) (end 48.514 96.08325) (width 0.2) (layer "F.Cu") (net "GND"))
 (segment (start 52.7 77.983) (end 52.7 75.05) (width 0.2) (layer "F.Cu") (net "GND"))
 (segment (start 45.0215 78.6765) (end 48.514 82.169) (width 0.2) (layer "F.Cu") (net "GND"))
 (segment (start 57.14425 104.39975) (end 56.8305 104.39975) (width 0.2) (layer "F.Cu") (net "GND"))
 (segment (start 74.93 72.39) (end 74.676 72.39) (width 0.2) (layer "F.Cu") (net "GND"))
 (via (at 74.93 72.39) (size 0.6) (drill 0.3) (layers "F.Cu" "B.Cu") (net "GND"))
 (via (at 45.0215 78.6765) (size 0.6) (drill 0.3) (layers "F.Cu" "B.Cu") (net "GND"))
 (segment (start 76.835 68.199) (end 70.866 62.23) (width 0.2) (layer "B.Cu") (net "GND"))
 (segment (start 44.196 77.851) (end 45.0215 78.6765) (width 0.2) (layer "B.Cu") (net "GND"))
 (segment (start 70.866 62.23) (end 54.356 62.23) (width 0.2) (layer "B.Cu") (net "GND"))
 (segment (start 74.93 72.39) (end 76.835 70.485) (width 0.2) (layer "B.Cu") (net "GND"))
 (segment (start 76.835 70.485) (end 76.835 68.199) (width 0.2) (layer "B.Cu") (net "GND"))
 (segment (start 44.196 72.39) (end 44.196 77.851) (width 0.2) (layer "B.Cu") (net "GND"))
 (segment (start 54.356 62.23) (end 44.196 72.39) (width 0.2) (layer "B.Cu") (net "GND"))
 (segment (start 54.55 76.45) (end 55.7 77.6) (width 0.2) (layer "F.Cu") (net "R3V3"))
 (segment (start 59.805 75.54175) (end 54.60825 75.54175) (width 0.2) (layer "F.Cu") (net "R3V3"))
 (segment (start 54.60825 75.54175) (end 54.55 75.6) (width 0.2) (layer "F.Cu") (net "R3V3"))
 (segment (start 54.55 75.6) (end 54.55 76.45) (width 0.2) (layer "F.Cu") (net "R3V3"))
 (via (at 55.7 77.6) (size 0.6) (drill 0.3) (layers "F.Cu" "B.Cu") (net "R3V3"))
 (segment (start 81.205 48.895) (end 87.63 48.895) (width 0.2) (layer "B.Cu") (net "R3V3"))
 (segment (start 56.05 77.95) (end 71.25 77.95) (width 0.2) (layer "B.Cu") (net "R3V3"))
 (segment (start 78.8 51.3) (end 81.205 48.895) (width 0.2) (layer "B.Cu") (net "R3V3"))
 (segment (start 71.25 77.95) (end 78.8 70.4) (width 0.2) (layer "B.Cu") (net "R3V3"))
 (segment (start 55.7 77.6) (end 56.05 77.95) (width 0.2) (layer "B.Cu") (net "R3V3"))
 (segment (start 78.8 70.4) (end 78.8 51.3) (width 0.2) (layer "B.Cu") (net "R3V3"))
 (segment (start 86.37 97.22) (end 84.5 99.09) (width 0.2) (layer "B.Cu") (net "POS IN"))
 (segment (start 86.37 90.6) (end 86.37 97.22) (width 0.2) (layer "B.Cu") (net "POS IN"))
 (segment (start 87.5 102.5) (end 84.64 102.5) (width 0.2) (layer "B.Cu") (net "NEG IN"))
 (segment (start 88.5 101.5) (end 87.5 102.5) (width 0.2) (layer "B.Cu") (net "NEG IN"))
 (segment (start 87.62 90.6) (end 88.5 91.48) (width 0.2) (layer "B.Cu") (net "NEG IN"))
 (segment (start 84.64 102.5) (end 84.5 102.64) (width 0.2) (layer "B.Cu") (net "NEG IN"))
 (segment (start 88.5 91.48) (end 88.5 101.5) (width 0.2) (layer "B.Cu") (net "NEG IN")))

